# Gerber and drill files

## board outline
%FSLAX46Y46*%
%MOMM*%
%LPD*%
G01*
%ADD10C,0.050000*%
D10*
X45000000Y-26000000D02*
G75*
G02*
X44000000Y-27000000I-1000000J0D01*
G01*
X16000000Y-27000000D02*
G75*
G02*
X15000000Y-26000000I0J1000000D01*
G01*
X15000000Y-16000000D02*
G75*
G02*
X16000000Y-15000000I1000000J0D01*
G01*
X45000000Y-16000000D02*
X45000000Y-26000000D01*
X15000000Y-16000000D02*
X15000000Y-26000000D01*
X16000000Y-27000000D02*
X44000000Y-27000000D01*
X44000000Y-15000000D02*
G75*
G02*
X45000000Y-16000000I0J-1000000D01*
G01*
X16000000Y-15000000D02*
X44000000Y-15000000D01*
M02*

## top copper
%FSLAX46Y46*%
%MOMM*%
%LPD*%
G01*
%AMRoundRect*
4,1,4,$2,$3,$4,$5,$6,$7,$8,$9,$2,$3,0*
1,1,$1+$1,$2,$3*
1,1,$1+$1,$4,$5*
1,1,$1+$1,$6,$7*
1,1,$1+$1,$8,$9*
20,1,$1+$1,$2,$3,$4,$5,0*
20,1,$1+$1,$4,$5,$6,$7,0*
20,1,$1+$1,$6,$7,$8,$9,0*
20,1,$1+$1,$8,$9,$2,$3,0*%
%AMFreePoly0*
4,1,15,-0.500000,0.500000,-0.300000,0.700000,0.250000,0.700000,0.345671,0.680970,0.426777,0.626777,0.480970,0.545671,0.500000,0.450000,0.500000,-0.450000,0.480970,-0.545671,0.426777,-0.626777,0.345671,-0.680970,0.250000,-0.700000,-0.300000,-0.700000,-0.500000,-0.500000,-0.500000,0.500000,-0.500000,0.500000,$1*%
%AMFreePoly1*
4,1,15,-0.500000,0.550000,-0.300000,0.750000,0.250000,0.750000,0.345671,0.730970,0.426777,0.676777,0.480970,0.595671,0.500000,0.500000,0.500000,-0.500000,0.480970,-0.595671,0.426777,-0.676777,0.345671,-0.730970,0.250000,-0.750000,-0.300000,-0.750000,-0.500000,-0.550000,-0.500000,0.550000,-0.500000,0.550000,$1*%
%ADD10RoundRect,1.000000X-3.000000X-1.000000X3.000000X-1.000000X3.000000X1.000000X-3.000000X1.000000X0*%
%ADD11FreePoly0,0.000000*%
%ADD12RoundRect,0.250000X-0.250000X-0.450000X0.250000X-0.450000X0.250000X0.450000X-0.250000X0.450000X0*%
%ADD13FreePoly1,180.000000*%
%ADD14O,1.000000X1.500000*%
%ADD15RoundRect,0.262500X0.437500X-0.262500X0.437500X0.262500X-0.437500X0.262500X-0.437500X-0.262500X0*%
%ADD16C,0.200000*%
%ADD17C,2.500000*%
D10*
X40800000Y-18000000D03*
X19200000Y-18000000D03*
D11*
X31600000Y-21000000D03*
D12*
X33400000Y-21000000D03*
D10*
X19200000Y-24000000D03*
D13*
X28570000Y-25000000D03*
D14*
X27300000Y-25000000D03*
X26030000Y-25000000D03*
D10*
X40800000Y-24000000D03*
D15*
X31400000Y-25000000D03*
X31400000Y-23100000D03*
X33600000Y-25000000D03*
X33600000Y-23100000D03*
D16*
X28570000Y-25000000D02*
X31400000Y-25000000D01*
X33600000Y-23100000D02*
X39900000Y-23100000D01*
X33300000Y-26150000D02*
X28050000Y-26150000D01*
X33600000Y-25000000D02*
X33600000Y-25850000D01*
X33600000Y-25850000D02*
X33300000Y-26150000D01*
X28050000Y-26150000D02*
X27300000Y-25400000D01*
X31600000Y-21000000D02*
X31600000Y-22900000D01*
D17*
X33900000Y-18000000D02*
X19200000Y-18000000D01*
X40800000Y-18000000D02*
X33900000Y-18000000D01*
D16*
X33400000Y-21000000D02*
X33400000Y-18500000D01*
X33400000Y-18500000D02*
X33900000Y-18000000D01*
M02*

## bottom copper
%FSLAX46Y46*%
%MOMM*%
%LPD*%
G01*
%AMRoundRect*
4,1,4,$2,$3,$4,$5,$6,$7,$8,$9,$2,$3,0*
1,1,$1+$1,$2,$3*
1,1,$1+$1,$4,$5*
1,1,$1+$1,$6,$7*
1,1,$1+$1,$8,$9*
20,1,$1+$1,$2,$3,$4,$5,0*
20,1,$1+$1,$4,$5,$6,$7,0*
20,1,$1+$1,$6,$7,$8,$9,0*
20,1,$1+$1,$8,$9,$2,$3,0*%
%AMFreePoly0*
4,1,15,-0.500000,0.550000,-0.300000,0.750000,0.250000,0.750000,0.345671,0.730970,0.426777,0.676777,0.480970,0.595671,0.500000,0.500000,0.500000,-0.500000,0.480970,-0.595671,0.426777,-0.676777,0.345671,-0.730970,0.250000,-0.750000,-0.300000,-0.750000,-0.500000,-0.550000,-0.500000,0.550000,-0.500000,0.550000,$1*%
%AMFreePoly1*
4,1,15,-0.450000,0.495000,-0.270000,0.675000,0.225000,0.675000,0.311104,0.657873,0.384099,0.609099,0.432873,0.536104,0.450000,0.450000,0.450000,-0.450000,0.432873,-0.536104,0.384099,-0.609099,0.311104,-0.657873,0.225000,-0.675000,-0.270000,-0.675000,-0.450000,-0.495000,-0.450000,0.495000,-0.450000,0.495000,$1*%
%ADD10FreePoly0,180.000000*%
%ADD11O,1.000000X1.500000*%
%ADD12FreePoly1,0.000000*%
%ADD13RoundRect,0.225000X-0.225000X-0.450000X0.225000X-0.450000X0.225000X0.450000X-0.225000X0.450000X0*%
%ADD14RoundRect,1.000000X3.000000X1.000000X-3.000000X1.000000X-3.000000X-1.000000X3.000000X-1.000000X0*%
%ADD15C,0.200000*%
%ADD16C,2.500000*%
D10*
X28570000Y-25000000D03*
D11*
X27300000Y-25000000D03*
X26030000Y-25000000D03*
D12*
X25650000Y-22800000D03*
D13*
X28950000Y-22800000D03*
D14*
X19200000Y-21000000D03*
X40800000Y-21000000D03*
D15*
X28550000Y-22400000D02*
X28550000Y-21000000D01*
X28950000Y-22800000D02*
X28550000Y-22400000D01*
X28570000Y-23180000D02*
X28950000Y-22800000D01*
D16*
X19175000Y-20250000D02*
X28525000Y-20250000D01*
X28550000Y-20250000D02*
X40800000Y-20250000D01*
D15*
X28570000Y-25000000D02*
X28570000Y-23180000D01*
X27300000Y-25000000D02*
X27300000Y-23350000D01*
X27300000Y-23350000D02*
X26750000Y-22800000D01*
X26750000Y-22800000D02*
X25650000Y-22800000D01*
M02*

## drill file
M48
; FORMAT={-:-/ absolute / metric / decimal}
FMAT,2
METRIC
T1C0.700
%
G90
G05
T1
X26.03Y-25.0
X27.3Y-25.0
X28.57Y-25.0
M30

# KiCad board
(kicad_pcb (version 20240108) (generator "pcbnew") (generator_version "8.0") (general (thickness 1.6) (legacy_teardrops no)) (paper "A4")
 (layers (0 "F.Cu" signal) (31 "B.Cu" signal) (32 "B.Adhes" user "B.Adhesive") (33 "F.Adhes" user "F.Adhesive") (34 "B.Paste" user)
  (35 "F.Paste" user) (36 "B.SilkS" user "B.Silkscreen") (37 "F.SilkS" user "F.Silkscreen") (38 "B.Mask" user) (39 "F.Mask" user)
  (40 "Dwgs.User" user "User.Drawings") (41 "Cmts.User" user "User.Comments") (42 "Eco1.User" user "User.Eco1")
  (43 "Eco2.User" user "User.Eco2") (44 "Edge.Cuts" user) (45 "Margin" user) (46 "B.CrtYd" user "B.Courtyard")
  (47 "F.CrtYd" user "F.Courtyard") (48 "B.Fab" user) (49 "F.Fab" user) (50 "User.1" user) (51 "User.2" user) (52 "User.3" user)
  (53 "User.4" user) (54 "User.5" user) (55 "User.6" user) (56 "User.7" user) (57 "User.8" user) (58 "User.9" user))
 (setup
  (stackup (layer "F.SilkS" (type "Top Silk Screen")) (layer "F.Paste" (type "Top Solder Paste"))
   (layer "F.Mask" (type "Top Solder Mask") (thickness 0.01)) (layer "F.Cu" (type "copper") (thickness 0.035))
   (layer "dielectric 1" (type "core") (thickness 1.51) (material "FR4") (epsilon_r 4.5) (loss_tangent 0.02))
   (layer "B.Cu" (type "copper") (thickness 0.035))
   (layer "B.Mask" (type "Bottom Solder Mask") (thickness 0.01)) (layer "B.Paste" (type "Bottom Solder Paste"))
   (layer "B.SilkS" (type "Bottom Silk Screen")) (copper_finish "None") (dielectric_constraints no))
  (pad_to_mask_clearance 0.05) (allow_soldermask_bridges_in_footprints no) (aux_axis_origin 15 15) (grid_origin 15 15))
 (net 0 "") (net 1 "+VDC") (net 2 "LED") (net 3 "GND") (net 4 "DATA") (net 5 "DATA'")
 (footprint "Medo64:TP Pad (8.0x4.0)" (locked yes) (layer "F.Cu") (at 40.8 18)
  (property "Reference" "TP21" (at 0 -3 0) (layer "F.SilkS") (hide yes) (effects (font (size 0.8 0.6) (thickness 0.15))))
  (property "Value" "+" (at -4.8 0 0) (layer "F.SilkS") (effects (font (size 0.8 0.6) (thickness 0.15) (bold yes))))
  (pad "1" smd roundrect (at 0 0) (size 8 4) (layers "F.Cu" "F.Mask") (roundrect_rratio 0.25) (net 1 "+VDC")))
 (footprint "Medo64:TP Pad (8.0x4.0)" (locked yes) (layer "F.Cu") (at 19.2 18)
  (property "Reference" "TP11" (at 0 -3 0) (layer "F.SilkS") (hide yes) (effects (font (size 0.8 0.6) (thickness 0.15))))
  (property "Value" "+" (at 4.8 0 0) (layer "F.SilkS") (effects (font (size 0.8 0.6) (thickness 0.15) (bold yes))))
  (pad "1" smd roundrect (at 0 0) (size 8 4) (layers "F.Cu" "F.Mask") (roundrect_rratio 0.25) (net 1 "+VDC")))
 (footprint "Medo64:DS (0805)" (layer "F.Cu") (at 32.5 21)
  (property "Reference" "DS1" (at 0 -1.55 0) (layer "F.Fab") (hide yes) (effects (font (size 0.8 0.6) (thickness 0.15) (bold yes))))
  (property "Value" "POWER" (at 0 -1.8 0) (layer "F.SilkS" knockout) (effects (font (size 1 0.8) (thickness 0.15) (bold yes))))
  (pad "1" smd roundrect (at -0.9 0) (size 1 1.4) (layers "F.Cu" "F.Paste" "F.Mask") (roundrect_rratio 0.25) (chamfer_ratio 0.2)
   (chamfer top_left bottom_left) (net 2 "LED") (thermal_bridge_angle 45))
  (pad "2" smd roundrect (at 0.9 0) (size 1 1.4) (layers "F.Cu" "F.Paste" "F.Mask") (roundrect_rratio 0.25) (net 1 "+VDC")
   (thermal_bridge_angle 45)))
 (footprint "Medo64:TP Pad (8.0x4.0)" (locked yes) (layer "F.Cu") (at 19.2 24)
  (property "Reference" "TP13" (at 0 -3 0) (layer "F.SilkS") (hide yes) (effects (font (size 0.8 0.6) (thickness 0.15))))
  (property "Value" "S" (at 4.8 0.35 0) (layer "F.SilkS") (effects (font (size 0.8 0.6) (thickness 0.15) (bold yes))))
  (pad "1" smd roundrect (at 0 0) (size 8 4) (layers "F.Cu" "F.Mask") (roundrect_rratio 0.25)))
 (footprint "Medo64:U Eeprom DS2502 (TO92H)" (layer "F.Cu") (at 27.3 25 180)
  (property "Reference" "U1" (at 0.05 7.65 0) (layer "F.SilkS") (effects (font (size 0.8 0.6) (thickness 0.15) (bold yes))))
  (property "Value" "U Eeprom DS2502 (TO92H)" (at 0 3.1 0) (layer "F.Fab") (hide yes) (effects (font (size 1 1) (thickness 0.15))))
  (pad "1" thru_hole roundrect (at -1.27 0 180) (size 1 1.5) (drill 0.7) (layers "*.Cu" "B.Mask") (remove_unused_layers no)
   (roundrect_rratio 0.25) (chamfer_ratio 0.2) (chamfer top_left bottom_left) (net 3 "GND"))
  (pad "2" thru_hole oval (at 0 0 180) (size 1 1.5) (drill 0.7) (layers "*.Cu" "B.Mask") (remove_unused_layers no) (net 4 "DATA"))
  (pad "3" thru_hole oval (at 1.27 0 180) (size 1 1.5) (drill 0.7) (layers "*.Cu" "B.Mask") (remove_unused_layers no)))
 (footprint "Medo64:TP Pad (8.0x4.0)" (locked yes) (layer "F.Cu") (at 40.8 24)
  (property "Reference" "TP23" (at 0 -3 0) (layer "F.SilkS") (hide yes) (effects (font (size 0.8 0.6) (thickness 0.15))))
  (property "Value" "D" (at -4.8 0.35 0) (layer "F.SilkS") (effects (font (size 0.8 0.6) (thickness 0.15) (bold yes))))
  (pad "1" smd roundrect (at 0 0) (size 8 4) (layers "F.Cu" "F.Mask") (roundrect_rratio 0.25) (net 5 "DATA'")))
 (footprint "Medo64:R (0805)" (layer "F.Cu") (at 31.4 24.05 90)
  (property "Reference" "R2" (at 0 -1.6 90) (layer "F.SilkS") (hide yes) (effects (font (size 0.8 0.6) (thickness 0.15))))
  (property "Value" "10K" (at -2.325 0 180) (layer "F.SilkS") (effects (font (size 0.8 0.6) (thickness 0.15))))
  (pad "1" smd roundrect (at -0.95 0 90) (size 1.05 1.4) (layers "F.Cu" "F.Paste" "F.Mask") (roundrect_rratio 0.25) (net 3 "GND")
   (thermal_bridge_angle 45))
  (pad "2" smd roundrect (at 0.95 0 90) (size 1.05 1.4) (layers "F.Cu" "F.Paste" "F.Mask") (roundrect_rratio 0.25) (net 2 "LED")
   (thermal_bridge_angle 45)))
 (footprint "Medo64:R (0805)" (layer "F.Cu") (at 33.6 24.05 90)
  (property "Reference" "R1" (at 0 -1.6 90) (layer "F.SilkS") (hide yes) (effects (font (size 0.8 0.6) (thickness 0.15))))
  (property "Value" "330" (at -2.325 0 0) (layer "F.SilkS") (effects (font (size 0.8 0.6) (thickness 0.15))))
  (pad "1" smd roundrect (at -0.95 0 90) (size 1.05 1.4) (layers "F.Cu" "F.Paste" "F.Mask") (roundrect_rratio 0.25) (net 4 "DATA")
   (thermal_bridge_angle 45))
  (pad "2" smd roundrect (at 0.95 0 90) (size 1.05 1.4) (layers "F.Cu" "F.Paste" "F.Mask") (roundrect_rratio 0.25) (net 5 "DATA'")
   (thermal_bridge_angle 45)))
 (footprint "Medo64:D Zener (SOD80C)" (layer "B.Cu") (at 27.3 22.8)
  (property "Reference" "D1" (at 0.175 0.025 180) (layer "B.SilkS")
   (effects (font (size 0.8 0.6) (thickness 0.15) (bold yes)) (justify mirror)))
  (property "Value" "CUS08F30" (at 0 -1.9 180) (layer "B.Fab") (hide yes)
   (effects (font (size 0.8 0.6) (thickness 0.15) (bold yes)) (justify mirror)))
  (pad "1" smd roundrect (at -1.65 0) (size 0.9 1.35) (layers "B.Cu" "B.Paste" "B.Mask") (roundrect_rratio 0.25) (chamfer_ratio 0.2)
   (chamfer top_left bottom_left) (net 4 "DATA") (thermal_bridge_angle 45))
  (pad "2" smd roundrect (at 1.65 0) (size 0.9 1.35) (layers "B.Cu" "B.Paste" "B.Mask") (roundrect_rratio 0.25) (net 3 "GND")
   (thermal_bridge_angle 45)))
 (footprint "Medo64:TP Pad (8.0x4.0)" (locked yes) (layer "B.Cu") (at 19.2 21 180)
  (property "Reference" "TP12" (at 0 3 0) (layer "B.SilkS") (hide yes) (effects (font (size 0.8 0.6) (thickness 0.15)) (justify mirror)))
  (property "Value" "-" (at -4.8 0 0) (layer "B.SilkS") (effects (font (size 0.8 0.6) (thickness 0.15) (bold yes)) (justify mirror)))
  (pad "1" smd roundrect (at 0 0 180) (size 8 4) (layers "B.Cu" "B.Mask") (roundrect_rratio 0.25) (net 3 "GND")))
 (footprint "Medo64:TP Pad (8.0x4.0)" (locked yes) (layer "B.Cu") (at 40.8 21 180)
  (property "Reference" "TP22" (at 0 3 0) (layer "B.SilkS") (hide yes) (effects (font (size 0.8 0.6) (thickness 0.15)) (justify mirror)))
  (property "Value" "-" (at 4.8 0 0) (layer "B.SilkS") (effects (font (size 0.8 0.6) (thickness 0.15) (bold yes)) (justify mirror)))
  (pad "1" smd roundrect (at 0 0 180) (size 8 4) (layers "B.Cu" "B.Mask") (roundrect_rratio 0.25) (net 3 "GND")))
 (gr_arc (start 45 26) (mid 44.707107 26.707107) (end 44 27) (locked yes) (stroke (width 0.05) (type default)) (layer "Edge.Cuts"))
 (gr_arc (start 16 27) (mid 15.292893 26.707107) (end 15 26) (locked yes) (stroke (width 0.05) (type default)) (layer "Edge.Cuts"))
 (gr_arc (start 15 16) (mid 15.292893 15.292893) (end 16 15) (locked yes) (stroke (width 0.05) (type default)) (layer "Edge.Cuts"))
 (gr_line (start 45 16) (end 45 26) (locked yes) (stroke (width 0.05) (type default)) (layer "Edge.Cuts"))
 (gr_line (start 15 16) (end 15 26) (locked yes) (stroke (width 0.05) (type default)) (layer "Edge.Cuts"))
 (gr_line (start 16 27) (end 44 27) (locked yes) (stroke (width 0.05) (type default)) (layer "Edge.Cuts"))
 (gr_arc (start 44 15) (mid 44.707107 15.292893) (end 45 16) (locked yes) (stroke (width 0.05) (type default)) (layer "Edge.Cuts"))
 (gr_line (start 16 15) (end 44 15) (locked yes) (stroke (width 0.05) (type default)) (layer "Edge.Cuts"))
 (segment (start 28.57 25) (end 31.4 25) (width 0.2) (layer "F.Cu") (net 3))
 (segment (start 28.55 22.4) (end 28.55 21) (width 0.2) (layer "B.Cu") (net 3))
 (segment (start 28.95 22.8) (end 28.55 22.4) (width 0.2) (layer "B.Cu") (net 3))
 (segment (start 28.57 23.18) (end 28.95 22.8) (width 0.2) (layer "B.Cu") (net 3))
 (segment (start 19.175 20.25) (end 28.525 20.25) (width 2.5) (layer "B.Cu") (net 3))
 (segment (start 28.55 20.25) (end 40.8 20.25) (width 2.5) (layer "B.Cu") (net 3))
 (segment (start 28.57 25) (end 28.57 23.18) (width 0.2) (layer "B.Cu") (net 3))
 (segment (start 33.6 23.1) (end 39.9 23.1) (width 0.2) (layer "F.Cu") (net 5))
 (segment (start 33.3 26.15) (end 28.05 26.15) (width 0.2) (layer "F.Cu") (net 4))
 (segment (start 33.6 25) (end 33.6 25.85) (width 0.2) (layer "F.Cu") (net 4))
 (segment (start 33.6 25.85) (end 33.3 26.15) (width 0.2) (layer "F.Cu") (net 4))
 (segment (start 28.05 26.15) (end 27.3 25.4) (width 0.2) (layer "F.Cu") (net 4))
 (segment (start 27.3 25) (end 27.3 23.35) (width 0.2) (layer "B.Cu") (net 4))
 (segment (start 27.3 23.35) (end 26.75 22.8) (width 0.2) (layer "B.Cu") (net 4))
 (segment (start 26.75 22.8) (end 25.65 22.8) (width 0.2) (layer "B.Cu") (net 4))
 (segment (start 31.6 21) (end 31.6 22.9) (width 0.2) (layer "F.Cu") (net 2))
 (segment (start 33.9 18) (end 19.2 18) (width 2.5) (layer "F.Cu") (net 1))
 (segment (start 40.8 18) (end 33.9 18) (width 2.5) (layer "F.Cu") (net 1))
 (segment (start 33.4 21) (end 33.4 18.5) (width 0.2) (layer "F.Cu") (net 1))
 (segment (start 33.4 18.5) (end 33.9 18) (width 0.2) (layer "F.Cu") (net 1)))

